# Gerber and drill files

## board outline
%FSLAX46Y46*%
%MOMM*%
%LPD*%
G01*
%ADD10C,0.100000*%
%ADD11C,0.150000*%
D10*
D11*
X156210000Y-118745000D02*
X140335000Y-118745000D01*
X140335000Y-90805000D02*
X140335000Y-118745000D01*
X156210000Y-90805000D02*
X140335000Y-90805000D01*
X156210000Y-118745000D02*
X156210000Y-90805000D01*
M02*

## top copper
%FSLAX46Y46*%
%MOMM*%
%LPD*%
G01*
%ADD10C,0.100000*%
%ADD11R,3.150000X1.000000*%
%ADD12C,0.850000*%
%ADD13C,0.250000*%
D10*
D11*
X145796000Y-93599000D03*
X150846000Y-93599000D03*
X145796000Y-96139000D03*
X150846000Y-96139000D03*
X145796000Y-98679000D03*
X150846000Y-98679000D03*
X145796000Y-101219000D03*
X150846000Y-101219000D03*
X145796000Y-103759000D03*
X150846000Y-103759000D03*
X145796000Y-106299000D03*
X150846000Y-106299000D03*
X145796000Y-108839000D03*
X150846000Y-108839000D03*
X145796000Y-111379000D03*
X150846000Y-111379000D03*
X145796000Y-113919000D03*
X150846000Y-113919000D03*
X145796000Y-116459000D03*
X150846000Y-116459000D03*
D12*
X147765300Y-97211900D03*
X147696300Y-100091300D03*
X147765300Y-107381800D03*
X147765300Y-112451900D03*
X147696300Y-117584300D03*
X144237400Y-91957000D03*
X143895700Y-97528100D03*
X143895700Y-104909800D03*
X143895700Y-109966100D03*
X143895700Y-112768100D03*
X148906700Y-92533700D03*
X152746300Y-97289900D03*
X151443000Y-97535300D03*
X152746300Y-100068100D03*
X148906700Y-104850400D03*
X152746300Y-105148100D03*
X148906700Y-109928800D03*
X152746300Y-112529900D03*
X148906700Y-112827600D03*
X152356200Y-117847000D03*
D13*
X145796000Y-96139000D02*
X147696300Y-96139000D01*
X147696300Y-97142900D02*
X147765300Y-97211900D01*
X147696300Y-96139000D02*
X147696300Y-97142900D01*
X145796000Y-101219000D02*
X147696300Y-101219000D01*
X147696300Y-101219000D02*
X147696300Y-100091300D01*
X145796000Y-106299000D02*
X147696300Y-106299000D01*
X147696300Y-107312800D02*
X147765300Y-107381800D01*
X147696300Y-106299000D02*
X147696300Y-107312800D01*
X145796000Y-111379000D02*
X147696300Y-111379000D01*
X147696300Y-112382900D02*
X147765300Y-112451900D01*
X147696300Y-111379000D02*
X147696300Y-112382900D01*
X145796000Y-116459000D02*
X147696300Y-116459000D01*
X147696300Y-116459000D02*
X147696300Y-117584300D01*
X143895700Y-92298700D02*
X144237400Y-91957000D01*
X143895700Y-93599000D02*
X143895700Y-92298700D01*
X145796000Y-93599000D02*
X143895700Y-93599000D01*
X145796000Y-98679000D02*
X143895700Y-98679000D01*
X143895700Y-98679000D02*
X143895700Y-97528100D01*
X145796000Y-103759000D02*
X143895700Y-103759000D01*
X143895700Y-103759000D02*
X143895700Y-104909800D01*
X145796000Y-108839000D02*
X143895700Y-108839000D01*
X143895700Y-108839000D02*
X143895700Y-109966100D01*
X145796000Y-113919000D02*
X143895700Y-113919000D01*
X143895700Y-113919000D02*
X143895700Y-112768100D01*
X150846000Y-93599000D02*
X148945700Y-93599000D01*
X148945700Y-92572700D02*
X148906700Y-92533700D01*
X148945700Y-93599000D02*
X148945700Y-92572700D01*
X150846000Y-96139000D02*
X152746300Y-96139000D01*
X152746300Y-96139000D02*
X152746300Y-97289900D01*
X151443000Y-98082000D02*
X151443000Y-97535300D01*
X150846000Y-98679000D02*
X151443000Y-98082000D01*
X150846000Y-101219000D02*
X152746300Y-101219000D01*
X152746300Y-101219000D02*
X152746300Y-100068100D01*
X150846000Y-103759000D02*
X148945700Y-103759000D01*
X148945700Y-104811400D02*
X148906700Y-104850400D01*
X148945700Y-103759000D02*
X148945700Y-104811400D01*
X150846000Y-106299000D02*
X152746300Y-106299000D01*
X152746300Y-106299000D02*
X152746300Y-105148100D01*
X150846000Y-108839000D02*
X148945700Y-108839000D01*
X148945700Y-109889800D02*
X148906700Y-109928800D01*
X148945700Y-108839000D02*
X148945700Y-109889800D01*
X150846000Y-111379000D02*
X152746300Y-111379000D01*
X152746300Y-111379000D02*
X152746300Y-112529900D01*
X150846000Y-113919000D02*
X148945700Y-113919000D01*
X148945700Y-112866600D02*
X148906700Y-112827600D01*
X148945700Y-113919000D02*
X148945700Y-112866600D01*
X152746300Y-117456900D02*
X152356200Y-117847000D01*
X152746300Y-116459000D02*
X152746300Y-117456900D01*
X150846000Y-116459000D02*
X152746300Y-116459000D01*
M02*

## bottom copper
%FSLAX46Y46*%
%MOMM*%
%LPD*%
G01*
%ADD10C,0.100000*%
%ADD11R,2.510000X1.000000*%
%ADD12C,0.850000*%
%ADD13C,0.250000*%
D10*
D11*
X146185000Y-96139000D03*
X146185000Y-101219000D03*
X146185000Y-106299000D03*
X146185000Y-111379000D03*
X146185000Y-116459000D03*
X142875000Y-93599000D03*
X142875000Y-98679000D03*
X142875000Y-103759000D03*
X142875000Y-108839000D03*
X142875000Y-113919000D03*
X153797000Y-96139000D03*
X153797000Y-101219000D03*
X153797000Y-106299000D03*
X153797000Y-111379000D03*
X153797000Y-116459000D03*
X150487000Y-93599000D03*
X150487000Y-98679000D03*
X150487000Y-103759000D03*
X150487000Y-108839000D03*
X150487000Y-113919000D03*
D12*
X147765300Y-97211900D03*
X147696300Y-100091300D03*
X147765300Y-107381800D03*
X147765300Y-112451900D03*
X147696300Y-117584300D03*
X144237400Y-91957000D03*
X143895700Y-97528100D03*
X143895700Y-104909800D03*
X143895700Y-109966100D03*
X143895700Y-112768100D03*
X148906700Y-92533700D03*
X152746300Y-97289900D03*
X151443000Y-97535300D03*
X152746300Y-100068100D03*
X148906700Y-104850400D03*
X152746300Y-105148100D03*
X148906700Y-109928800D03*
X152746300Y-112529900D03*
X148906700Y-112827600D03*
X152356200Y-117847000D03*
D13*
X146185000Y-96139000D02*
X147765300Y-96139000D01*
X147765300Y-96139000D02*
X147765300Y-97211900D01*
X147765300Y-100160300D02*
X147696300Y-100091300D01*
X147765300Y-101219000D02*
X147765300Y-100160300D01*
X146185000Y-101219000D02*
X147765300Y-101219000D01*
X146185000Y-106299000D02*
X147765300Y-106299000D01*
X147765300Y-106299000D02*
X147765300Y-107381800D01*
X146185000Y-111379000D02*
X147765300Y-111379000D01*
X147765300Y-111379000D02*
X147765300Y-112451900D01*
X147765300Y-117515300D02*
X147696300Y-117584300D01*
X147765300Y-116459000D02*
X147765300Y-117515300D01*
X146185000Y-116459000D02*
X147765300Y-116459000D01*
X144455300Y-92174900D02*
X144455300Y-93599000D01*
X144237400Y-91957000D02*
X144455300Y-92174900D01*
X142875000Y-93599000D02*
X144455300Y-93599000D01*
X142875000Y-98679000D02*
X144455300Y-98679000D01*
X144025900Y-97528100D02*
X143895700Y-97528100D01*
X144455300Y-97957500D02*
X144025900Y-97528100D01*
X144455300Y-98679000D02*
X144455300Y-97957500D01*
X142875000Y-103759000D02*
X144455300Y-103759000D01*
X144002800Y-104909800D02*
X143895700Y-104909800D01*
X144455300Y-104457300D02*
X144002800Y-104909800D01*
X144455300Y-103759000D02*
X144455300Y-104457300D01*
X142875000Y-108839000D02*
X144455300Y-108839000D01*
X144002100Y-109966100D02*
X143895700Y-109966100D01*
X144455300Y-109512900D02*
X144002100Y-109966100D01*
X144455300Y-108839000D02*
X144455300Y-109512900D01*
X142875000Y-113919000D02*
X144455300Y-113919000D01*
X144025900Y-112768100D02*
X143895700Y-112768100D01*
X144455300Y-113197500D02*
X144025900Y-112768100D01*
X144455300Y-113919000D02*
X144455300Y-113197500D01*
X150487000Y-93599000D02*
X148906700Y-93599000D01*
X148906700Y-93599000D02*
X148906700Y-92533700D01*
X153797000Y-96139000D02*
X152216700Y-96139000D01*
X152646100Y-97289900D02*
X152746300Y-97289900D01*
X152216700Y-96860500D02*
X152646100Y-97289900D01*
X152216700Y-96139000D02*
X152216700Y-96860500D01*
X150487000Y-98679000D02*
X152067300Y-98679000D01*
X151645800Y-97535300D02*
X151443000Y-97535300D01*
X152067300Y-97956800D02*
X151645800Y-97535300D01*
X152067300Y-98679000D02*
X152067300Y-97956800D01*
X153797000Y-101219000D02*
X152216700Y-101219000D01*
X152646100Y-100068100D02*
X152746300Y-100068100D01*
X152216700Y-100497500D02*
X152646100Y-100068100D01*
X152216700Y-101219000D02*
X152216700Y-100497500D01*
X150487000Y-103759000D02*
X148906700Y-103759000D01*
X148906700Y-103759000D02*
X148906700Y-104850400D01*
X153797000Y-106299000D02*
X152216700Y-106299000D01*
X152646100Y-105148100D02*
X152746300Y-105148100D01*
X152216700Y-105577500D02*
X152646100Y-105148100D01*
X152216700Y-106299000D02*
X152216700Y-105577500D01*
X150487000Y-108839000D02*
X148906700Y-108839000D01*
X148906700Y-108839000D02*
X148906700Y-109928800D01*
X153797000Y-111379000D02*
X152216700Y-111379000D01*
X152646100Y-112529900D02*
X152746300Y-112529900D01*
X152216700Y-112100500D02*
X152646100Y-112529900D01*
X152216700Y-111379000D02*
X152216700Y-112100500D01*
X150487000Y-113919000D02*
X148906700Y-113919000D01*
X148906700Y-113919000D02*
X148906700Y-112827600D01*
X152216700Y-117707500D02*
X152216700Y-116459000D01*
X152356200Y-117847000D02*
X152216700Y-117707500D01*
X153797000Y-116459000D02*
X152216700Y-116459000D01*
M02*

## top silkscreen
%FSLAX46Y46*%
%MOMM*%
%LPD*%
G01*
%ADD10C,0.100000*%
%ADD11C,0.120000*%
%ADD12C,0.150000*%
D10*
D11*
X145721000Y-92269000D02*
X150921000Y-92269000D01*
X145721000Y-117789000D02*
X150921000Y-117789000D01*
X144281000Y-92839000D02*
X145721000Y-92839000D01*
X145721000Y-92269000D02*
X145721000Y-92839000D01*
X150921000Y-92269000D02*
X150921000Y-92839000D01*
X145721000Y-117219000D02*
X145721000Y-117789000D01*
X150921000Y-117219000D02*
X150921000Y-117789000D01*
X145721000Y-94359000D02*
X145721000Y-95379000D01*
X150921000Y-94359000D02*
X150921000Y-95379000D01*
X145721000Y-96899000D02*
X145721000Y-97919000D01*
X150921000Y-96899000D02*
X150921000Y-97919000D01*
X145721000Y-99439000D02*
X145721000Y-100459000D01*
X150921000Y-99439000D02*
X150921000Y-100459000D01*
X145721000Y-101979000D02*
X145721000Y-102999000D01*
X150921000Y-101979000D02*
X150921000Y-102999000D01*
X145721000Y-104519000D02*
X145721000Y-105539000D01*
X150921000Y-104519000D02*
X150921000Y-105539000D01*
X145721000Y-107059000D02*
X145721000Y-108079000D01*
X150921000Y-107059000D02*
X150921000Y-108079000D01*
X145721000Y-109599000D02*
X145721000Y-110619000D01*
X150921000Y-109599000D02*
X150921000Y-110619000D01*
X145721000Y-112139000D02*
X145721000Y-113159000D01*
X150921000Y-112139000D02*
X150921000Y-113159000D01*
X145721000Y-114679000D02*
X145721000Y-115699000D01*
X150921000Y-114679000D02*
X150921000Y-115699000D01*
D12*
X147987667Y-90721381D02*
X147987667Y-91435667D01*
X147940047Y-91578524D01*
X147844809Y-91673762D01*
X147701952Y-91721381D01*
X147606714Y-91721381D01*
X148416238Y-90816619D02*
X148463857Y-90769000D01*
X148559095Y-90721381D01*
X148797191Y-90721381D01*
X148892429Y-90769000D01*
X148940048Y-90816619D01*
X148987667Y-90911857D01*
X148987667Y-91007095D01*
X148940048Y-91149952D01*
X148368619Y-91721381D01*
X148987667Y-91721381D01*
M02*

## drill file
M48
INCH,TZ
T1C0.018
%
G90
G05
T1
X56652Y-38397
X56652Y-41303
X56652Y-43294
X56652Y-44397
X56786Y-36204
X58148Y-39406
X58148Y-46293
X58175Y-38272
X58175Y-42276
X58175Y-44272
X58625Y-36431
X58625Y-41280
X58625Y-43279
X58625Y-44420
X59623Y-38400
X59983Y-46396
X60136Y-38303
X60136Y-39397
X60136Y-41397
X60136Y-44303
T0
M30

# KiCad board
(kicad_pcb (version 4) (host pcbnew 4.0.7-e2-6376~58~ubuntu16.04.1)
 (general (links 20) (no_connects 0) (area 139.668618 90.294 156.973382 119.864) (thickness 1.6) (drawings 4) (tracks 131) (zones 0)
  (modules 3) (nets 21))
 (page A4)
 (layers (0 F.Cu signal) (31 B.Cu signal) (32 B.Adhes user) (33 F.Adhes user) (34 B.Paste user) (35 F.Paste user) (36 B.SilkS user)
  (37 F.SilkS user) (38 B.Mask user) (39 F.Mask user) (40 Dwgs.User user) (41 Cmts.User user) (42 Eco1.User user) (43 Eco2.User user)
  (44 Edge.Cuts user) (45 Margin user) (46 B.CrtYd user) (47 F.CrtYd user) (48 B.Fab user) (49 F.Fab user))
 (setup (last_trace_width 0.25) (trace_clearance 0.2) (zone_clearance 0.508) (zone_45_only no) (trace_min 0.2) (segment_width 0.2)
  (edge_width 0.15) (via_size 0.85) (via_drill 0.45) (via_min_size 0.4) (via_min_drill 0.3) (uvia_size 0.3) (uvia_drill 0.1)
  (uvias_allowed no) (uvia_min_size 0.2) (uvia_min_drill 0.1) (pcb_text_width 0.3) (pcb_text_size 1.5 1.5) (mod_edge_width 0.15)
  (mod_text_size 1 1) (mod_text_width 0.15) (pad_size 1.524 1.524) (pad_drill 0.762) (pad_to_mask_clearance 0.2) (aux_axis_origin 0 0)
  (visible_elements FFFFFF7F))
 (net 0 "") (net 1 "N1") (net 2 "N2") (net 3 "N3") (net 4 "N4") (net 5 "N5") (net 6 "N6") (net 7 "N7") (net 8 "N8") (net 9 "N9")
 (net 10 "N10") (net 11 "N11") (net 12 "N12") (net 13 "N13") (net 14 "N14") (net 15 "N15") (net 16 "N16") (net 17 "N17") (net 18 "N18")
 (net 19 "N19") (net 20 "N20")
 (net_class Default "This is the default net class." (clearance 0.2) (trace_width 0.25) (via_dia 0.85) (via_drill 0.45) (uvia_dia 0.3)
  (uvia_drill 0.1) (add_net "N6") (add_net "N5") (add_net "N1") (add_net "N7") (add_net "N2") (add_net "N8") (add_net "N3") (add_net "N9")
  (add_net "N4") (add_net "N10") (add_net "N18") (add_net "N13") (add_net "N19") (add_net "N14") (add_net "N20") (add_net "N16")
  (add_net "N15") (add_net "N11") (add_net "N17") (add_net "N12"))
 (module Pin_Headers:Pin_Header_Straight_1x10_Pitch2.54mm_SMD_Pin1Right (layer B.Cu) (at 144.53 105.029 180)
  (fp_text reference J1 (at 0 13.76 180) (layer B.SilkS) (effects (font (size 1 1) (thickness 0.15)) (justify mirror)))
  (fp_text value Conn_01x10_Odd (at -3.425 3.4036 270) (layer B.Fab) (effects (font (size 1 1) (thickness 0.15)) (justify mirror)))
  (pad 2 smd rect (at -1.655 8.89 180) (size 2.51 1) (layers B.Cu B.Paste B.Mask) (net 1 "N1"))
  (pad 4 smd rect (at -1.655 3.81 180) (size 2.51 1) (layers B.Cu B.Paste B.Mask) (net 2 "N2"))
  (pad 6 smd rect (at -1.655 -1.27 180) (size 2.51 1) (layers B.Cu B.Paste B.Mask) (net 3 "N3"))
  (pad 8 smd rect (at -1.655 -6.35 180) (size 2.51 1) (layers B.Cu B.Paste B.Mask) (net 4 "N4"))
  (pad 10 smd rect (at -1.655 -11.43 180) (size 2.51 1) (layers B.Cu B.Paste B.Mask) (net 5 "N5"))
  (pad 1 smd rect (at 1.655 11.43 180) (size 2.51 1) (layers B.Cu B.Paste B.Mask) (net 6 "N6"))
  (pad 3 smd rect (at 1.655 6.35 180) (size 2.51 1) (layers B.Cu B.Paste B.Mask) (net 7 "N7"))
  (pad 5 smd rect (at 1.655 1.27 180) (size 2.51 1) (layers B.Cu B.Paste B.Mask) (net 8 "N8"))
  (pad 7 smd rect (at 1.655 -3.81 180) (size 2.51 1) (layers B.Cu B.Paste B.Mask) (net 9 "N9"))
  (pad 9 smd rect (at 1.655 -8.89 180) (size 2.51 1) (layers B.Cu B.Paste B.Mask) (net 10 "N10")))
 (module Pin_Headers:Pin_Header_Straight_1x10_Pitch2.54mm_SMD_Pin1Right (layer B.Cu) (at 152.142 105.029 180)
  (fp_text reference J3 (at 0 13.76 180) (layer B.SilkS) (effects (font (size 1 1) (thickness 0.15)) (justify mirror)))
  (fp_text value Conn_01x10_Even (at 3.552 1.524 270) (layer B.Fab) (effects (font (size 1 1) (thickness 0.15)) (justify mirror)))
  (pad 2 smd rect (at -1.655 8.89 180) (size 2.51 1) (layers B.Cu B.Paste B.Mask) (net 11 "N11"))
  (pad 4 smd rect (at -1.655 3.81 180) (size 2.51 1) (layers B.Cu B.Paste B.Mask) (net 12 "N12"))
  (pad 6 smd rect (at -1.655 -1.27 180) (size 2.51 1) (layers B.Cu B.Paste B.Mask) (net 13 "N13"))
  (pad 8 smd rect (at -1.655 -6.35 180) (size 2.51 1) (layers B.Cu B.Paste B.Mask) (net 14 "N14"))
  (pad 10 smd rect (at -1.655 -11.43 180) (size 2.51 1) (layers B.Cu B.Paste B.Mask) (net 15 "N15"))
  (pad 1 smd rect (at 1.655 11.43 180) (size 2.51 1) (layers B.Cu B.Paste B.Mask) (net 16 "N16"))
  (pad 3 smd rect (at 1.655 6.35 180) (size 2.51 1) (layers B.Cu B.Paste B.Mask) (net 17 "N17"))
  (pad 5 smd rect (at 1.655 1.27 180) (size 2.51 1) (layers B.Cu B.Paste B.Mask) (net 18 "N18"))
  (pad 7 smd rect (at 1.655 -3.81 180) (size 2.51 1) (layers B.Cu B.Paste B.Mask) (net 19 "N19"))
  (pad 9 smd rect (at 1.655 -8.89 180) (size 2.51 1) (layers B.Cu B.Paste B.Mask) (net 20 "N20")))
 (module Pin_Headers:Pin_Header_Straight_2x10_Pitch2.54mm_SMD (layer F.Cu) (at 148.321 105.029)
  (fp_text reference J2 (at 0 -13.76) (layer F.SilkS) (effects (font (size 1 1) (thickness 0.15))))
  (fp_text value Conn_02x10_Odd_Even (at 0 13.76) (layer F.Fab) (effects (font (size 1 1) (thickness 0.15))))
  (fp_line (start -2.6 -12.76) (end 2.6 -12.76) (layer F.SilkS) (width 0.12))
  (fp_line (start -2.6 12.76) (end 2.6 12.76) (layer F.SilkS) (width 0.12))
  (fp_line (start -4.04 -12.19) (end -2.6 -12.19) (layer F.SilkS) (width 0.12))
  (fp_line (start -2.6 -12.76) (end -2.6 -12.19) (layer F.SilkS) (width 0.12))
  (fp_line (start 2.6 -12.76) (end 2.6 -12.19) (layer F.SilkS) (width 0.12))
  (fp_line (start -2.6 12.19) (end -2.6 12.76) (layer F.SilkS) (width 0.12))
  (fp_line (start 2.6 12.19) (end 2.6 12.76) (layer F.SilkS) (width 0.12))
  (fp_line (start -2.6 -10.67) (end -2.6 -9.65) (layer F.SilkS) (width 0.12))
  (fp_line (start 2.6 -10.67) (end 2.6 -9.65) (layer F.SilkS) (width 0.12))
  (fp_line (start -2.6 -8.13) (end -2.6 -7.11) (layer F.SilkS) (width 0.12))
  (fp_line (start 2.6 -8.13) (end 2.6 -7.11) (layer F.SilkS) (width 0.12))
  (fp_line (start -2.6 -5.59) (end -2.6 -4.57) (layer F.SilkS) (width 0.12))
  (fp_line (start 2.6 -5.59) (end 2.6 -4.57) (layer F.SilkS) (width 0.12))
  (fp_line (start -2.6 -3.05) (end -2.6 -2.03) (layer F.SilkS) (width 0.12))
  (fp_line (start 2.6 -3.05) (end 2.6 -2.03) (layer F.SilkS) (width 0.12))
  (fp_line (start -2.6 -0.51) (end -2.6 0.51) (layer F.SilkS) (width 0.12))
  (fp_line (start 2.6 -0.51) (end 2.6 0.51) (layer F.SilkS) (width 0.12))
  (fp_line (start -2.6 2.03) (end -2.6 3.05) (layer F.SilkS) (width 0.12))
  (fp_line (start 2.6 2.03) (end 2.6 3.05) (layer F.SilkS) (width 0.12))
  (fp_line (start -2.6 4.57) (end -2.6 5.59) (layer F.SilkS) (width 0.12))
  (fp_line (start 2.6 4.57) (end 2.6 5.59) (layer F.SilkS) (width 0.12))
  (fp_line (start -2.6 7.11) (end -2.6 8.13) (layer F.SilkS) (width 0.12))
  (fp_line (start 2.6 7.11) (end 2.6 8.13) (layer F.SilkS) (width 0.12))
  (fp_line (start -2.6 9.65) (end -2.6 10.67) (layer F.SilkS) (width 0.12))
  (fp_line (start 2.6 9.65) (end 2.6 10.67) (layer F.SilkS) (width 0.12))
  (pad 1 smd rect (at -2.525 -11.43) (size 3.15 1) (layers F.Cu F.Paste F.Mask) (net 6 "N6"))
  (pad 2 smd rect (at 2.525 -11.43) (size 3.15 1) (layers F.Cu F.Paste F.Mask) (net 16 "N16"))
  (pad 3 smd rect (at -2.525 -8.89) (size 3.15 1) (layers F.Cu F.Paste F.Mask) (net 1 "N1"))
  (pad 4 smd rect (at 2.525 -8.89) (size 3.15 1) (layers F.Cu F.Paste F.Mask) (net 11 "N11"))
  (pad 5 smd rect (at -2.525 -6.35) (size 3.15 1) (layers F.Cu F.Paste F.Mask) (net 7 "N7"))
  (pad 6 smd rect (at 2.525 -6.35) (size 3.15 1) (layers F.Cu F.Paste F.Mask) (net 17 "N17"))
  (pad 7 smd rect (at -2.525 -3.81) (size 3.15 1) (layers F.Cu F.Paste F.Mask) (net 2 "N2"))
  (pad 8 smd rect (at 2.525 -3.81) (size 3.15 1) (layers F.Cu F.Paste F.Mask) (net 12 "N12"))
  (pad 9 smd rect (at -2.525 -1.27) (size 3.15 1) (layers F.Cu F.Paste F.Mask) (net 8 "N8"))
  (pad 10 smd rect (at 2.525 -1.27) (size 3.15 1) (layers F.Cu F.Paste F.Mask) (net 18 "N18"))
  (pad 11 smd rect (at -2.525 1.27) (size 3.15 1) (layers F.Cu F.Paste F.Mask) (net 3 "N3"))
  (pad 12 smd rect (at 2.525 1.27) (size 3.15 1) (layers F.Cu F.Paste F.Mask) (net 13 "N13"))
  (pad 13 smd rect (at -2.525 3.81) (size 3.15 1) (layers F.Cu F.Paste F.Mask) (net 9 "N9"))
  (pad 14 smd rect (at 2.525 3.81) (size 3.15 1) (layers F.Cu F.Paste F.Mask) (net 19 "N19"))
  (pad 15 smd rect (at -2.525 6.35) (size 3.15 1) (layers F.Cu F.Paste F.Mask) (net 4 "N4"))
  (pad 16 smd rect (at 2.525 6.35) (size 3.15 1) (layers F.Cu F.Paste F.Mask) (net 14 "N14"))
  (pad 17 smd rect (at -2.525 8.89) (size 3.15 1) (layers F.Cu F.Paste F.Mask) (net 10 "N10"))
  (pad 18 smd rect (at 2.525 8.89) (size 3.15 1) (layers F.Cu F.Paste F.Mask) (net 20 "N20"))
  (pad 19 smd rect (at -2.525 11.43) (size 3.15 1) (layers F.Cu F.Paste F.Mask) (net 5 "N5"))
  (pad 20 smd rect (at 2.525 11.43) (size 3.15 1) (layers F.Cu F.Paste F.Mask) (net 15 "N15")))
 (gr_line (start 156.21 118.745) (end 140.335 118.745) (layer Edge.Cuts) (width 0.15))
 (gr_line (start 140.335 90.805) (end 140.335 118.745) (layer Edge.Cuts) (width 0.15))
 (gr_line (start 156.21 90.805) (end 140.335 90.805) (layer Edge.Cuts) (width 0.15))
 (gr_line (start 156.21 118.745) (end 156.21 90.805) (layer Edge.Cuts) (width 0.15))
 (via (at 147.7653 97.2119) (size 0.85) (layers F.Cu B.Cu) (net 1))
 (segment (start 145.796 96.139) (end 147.6963 96.139) (width 0.25) (layer F.Cu) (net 1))
 (segment (start 146.185 96.139) (end 147.7653 96.139) (width 0.25) (layer B.Cu) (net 1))
 (segment (start 147.7653 96.139) (end 147.7653 97.2119) (width 0.25) (layer B.Cu) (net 1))
 (segment (start 147.6963 97.1429) (end 147.7653 97.2119) (width 0.25) (layer F.Cu) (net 1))
 (segment (start 147.6963 96.139) (end 147.6963 97.1429) (width 0.25) (layer F.Cu) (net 1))
 (via (at 147.6963 100.0913) (size 0.85) (layers F.Cu B.Cu) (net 2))
 (segment (start 145.796 101.219) (end 147.6963 101.219) (width 0.25) (layer F.Cu) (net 2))
 (segment (start 147.7653 100.1603) (end 147.6963 100.0913) (width 0.25) (layer B.Cu) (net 2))
 (segment (start 147.7653 101.219) (end 147.7653 100.1603) (width 0.25) (layer B.Cu) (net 2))
 (segment (start 147.6963 101.219) (end 147.6963 100.0913) (width 0.25) (layer F.Cu) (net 2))
 (segment (start 146.185 101.219) (end 147.7653 101.219) (width 0.25) (layer B.Cu) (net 2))
 (via (at 147.7653 107.3818) (size 0.85) (layers F.Cu B.Cu) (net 3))
 (segment (start 145.796 106.299) (end 147.6963 106.299) (width 0.25) (layer F.Cu) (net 3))
 (segment (start 146.185 106.299) (end 147.7653 106.299) (width 0.25) (layer B.Cu) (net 3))
 (segment (start 147.7653 106.299) (end 147.7653 107.3818) (width 0.25) (layer B.Cu) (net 3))
 (segment (start 147.6963 107.3128) (end 147.7653 107.3818) (width 0.25) (layer F.Cu) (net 3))
 (segment (start 147.6963 106.299) (end 147.6963 107.3128) (width 0.25) (layer F.Cu) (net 3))
 (via (at 147.7653 112.4519) (size 0.85) (layers F.Cu B.Cu) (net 4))
 (segment (start 145.796 111.379) (end 147.6963 111.379) (width 0.25) (layer F.Cu) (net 4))
 (segment (start 146.185 111.379) (end 147.7653 111.379) (width 0.25) (layer B.Cu) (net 4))
 (segment (start 147.7653 111.379) (end 147.7653 112.4519) (width 0.25) (layer B.Cu) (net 4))
 (segment (start 147.6963 112.3829) (end 147.7653 112.4519) (width 0.25) (layer F.Cu) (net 4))
 (segment (start 147.6963 111.379) (end 147.6963 112.3829) (width 0.25) (layer F.Cu) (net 4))
 (via (at 147.6963 117.5843) (size 0.85) (layers F.Cu B.Cu) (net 5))
 (segment (start 145.796 116.459) (end 147.6963 116.459) (width 0.25) (layer F.Cu) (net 5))
 (segment (start 147.7653 117.5153) (end 147.6963 117.5843) (width 0.25) (layer B.Cu) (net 5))
 (segment (start 147.7653 116.459) (end 147.7653 117.5153) (width 0.25) (layer B.Cu) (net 5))
 (segment (start 147.6963 116.459) (end 147.6963 117.5843) (width 0.25) (layer F.Cu) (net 5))
 (segment (start 146.185 116.459) (end 147.7653 116.459) (width 0.25) (layer B.Cu) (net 5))
 (via (at 144.2374 91.957) (size 0.85) (layers F.Cu B.Cu) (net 6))
 (segment (start 143.8957 92.2987) (end 144.2374 91.957) (width 0.25) (layer F.Cu) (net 6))
 (segment (start 143.8957 93.599) (end 143.8957 92.2987) (width 0.25) (layer F.Cu) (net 6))
 (segment (start 144.4553 92.1749) (end 144.4553 93.599) (width 0.25) (layer B.Cu) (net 6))
 (segment (start 144.2374 91.957) (end 144.4553 92.1749) (width 0.25) (layer B.Cu) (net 6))
 (segment (start 145.796 93.599) (end 143.8957 93.599) (width 0.25) (layer F.Cu) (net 6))
 (segment (start 142.875 93.599) (end 144.4553 93.599) (width 0.25) (layer B.Cu) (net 6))
 (via (at 143.8957 97.5281) (size 0.85) (layers F.Cu B.Cu) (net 7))
 (segment (start 145.796 98.679) (end 143.8957 98.679) (width 0.25) (layer F.Cu) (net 7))
 (segment (start 142.875 98.679) (end 144.4553 98.679) (width 0.25) (layer B.Cu) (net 7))
 (segment (start 144.0259 97.5281) (end 143.8957 97.5281) (width 0.25) (layer B.Cu) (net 7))
 (segment (start 144.4553 97.9575) (end 144.0259 97.5281) (width 0.25) (layer B.Cu) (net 7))
 (segment (start 144.4553 98.679) (end 144.4553 97.9575) (width 0.25) (layer B.Cu) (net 7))
 (segment (start 143.8957 98.679) (end 143.8957 97.5281) (width 0.25) (layer F.Cu) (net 7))
 (via (at 143.8957 104.9098) (size 0.85) (layers F.Cu B.Cu) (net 8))
 (segment (start 145.796 103.759) (end 143.8957 103.759) (width 0.25) (layer F.Cu) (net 8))
 (segment (start 142.875 103.759) (end 144.4553 103.759) (width 0.25) (layer B.Cu) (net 8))
 (segment (start 144.0028 104.9098) (end 143.8957 104.9098) (width 0.25) (layer B.Cu) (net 8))
 (segment (start 144.4553 104.4573) (end 144.0028 104.9098) (width 0.25) (layer B.Cu) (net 8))
 (segment (start 144.4553 103.759) (end 144.4553 104.4573) (width 0.25) (layer B.Cu) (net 8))
 (segment (start 143.8957 103.759) (end 143.8957 104.9098) (width 0.25) (layer F.Cu) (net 8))
 (via (at 143.8957 109.9661) (size 0.85) (layers F.Cu B.Cu) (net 9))
 (segment (start 145.796 108.839) (end 143.8957 108.839) (width 0.25) (layer F.Cu) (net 9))
 (segment (start 142.875 108.839) (end 144.4553 108.839) (width 0.25) (layer B.Cu) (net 9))
 (segment (start 144.0021 109.9661) (end 143.8957 109.9661) (width 0.25) (layer B.Cu) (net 9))
 (segment (start 144.4553 109.5129) (end 144.0021 109.9661) (width 0.25) (layer B.Cu) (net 9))
 (segment (start 144.4553 108.839) (end 144.4553 109.5129) (width 0.25) (layer B.Cu) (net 9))
 (segment (start 143.8957 108.839) (end 143.8957 109.9661) (width 0.25) (layer F.Cu) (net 9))
 (via (at 143.8957 112.7681) (size 0.85) (layers F.Cu B.Cu) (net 10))
 (segment (start 145.796 113.919) (end 143.8957 113.919) (width 0.25) (layer F.Cu) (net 10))
 (segment (start 142.875 113.919) (end 144.4553 113.919) (width 0.25) (layer B.Cu) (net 10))
 (segment (start 144.0259 112.7681) (end 143.8957 112.7681) (width 0.25) (layer B.Cu) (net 10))
 (segment (start 144.4553 113.1975) (end 144.0259 112.7681) (width 0.25) (layer B.Cu) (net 10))
 (segment (start 144.4553 113.919) (end 144.4553 113.1975) (width 0.25) (layer B.Cu) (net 10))
 (segment (start 143.8957 113.919) (end 143.8957 112.7681) (width 0.25) (layer F.Cu) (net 10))
 (via (at 148.9067 92.5337) (size 0.85) (layers F.Cu B.Cu) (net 16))
 (segment (start 150.846 93.599) (end 148.9457 93.599) (width 0.25) (layer F.Cu) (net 16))
 (segment (start 150.487 93.599) (end 148.9067 93.599) (width 0.25) (layer B.Cu) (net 16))
 (segment (start 148.9067 93.599) (end 148.9067 92.5337) (width 0.25) (layer B.Cu) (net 16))
 (segment (start 148.9457 92.5727) (end 148.9067 92.5337) (width 0.25) (layer F.Cu) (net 16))
 (segment (start 148.9457 93.599) (end 148.9457 92.5727) (width 0.25) (layer F.Cu) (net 16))
 (via (at 152.7463 97.2899) (size 0.85) (layers F.Cu B.Cu) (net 11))
 (segment (start 150.846 96.139) (end 152.7463 96.139) (width 0.25) (layer F.Cu) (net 11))
 (segment (start 153.797 96.139) (end 152.2167 96.139) (width 0.25) (layer B.Cu) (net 11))
 (segment (start 152.6461 97.2899) (end 152.7463 97.2899) (width 0.25) (layer B.Cu) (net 11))
 (segment (start 152.2167 96.8605) (end 152.6461 97.2899) (width 0.25) (layer B.Cu) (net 11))
 (segment (start 152.2167 96.139) (end 152.2167 96.8605) (width 0.25) (layer B.Cu) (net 11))
 (segment (start 152.7463 96.139) (end 152.7463 97.2899) (width 0.25) (layer F.Cu) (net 11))
 (via (at 151.443 97.5353) (size 0.85) (layers F.Cu B.Cu) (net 17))
 (segment (start 150.487 98.679) (end 152.0673 98.679) (width 0.25) (layer B.Cu) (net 17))
 (segment (start 151.6458 97.5353) (end 151.443 97.5353) (width 0.25) (layer B.Cu) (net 17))
 (segment (start 152.0673 97.9568) (end 151.6458 97.5353) (width 0.25) (layer B.Cu) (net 17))
 (segment (start 152.0673 98.679) (end 152.0673 97.9568) (width 0.25) (layer B.Cu) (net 17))
 (segment (start 151.443 98.082) (end 151.443 97.5353) (width 0.25) (layer F.Cu) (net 17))
 (segment (start 150.846 98.679) (end 151.443 98.082) (width 0.25) (layer F.Cu) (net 17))
 (via (at 152.7463 100.0681) (size 0.85) (layers F.Cu B.Cu) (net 12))
 (segment (start 150.846 101.219) (end 152.7463 101.219) (width 0.25) (layer F.Cu) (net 12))
 (segment (start 153.797 101.219) (end 152.2167 101.219) (width 0.25) (layer B.Cu) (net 12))
 (segment (start 152.6461 100.0681) (end 152.7463 100.0681) (width 0.25) (layer B.Cu) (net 12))
 (segment (start 152.2167 100.4975) (end 152.6461 100.0681) (width 0.25) (layer B.Cu) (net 12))
 (segment (start 152.2167 101.219) (end 152.2167 100.4975) (width 0.25) (layer B.Cu) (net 12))
 (segment (start 152.7463 101.219) (end 152.7463 100.0681) (width 0.25) (layer F.Cu) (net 12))
 (via (at 148.9067 104.8504) (size 0.85) (layers F.Cu B.Cu) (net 18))
 (segment (start 150.846 103.759) (end 148.9457 103.759) (width 0.25) (layer F.Cu) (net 18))
 (segment (start 150.487 103.759) (end 148.9067 103.759) (width 0.25) (layer B.Cu) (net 18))
 (segment (start 148.9067 103.759) (end 148.9067 104.8504) (width 0.25) (layer B.Cu) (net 18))
 (segment (start 148.9457 104.8114) (end 148.9067 104.8504) (width 0.25) (layer F.Cu) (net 18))
 (segment (start 148.9457 103.759) (end 148.9457 104.8114) (width 0.25) (layer F.Cu) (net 18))
 (via (at 152.7463 105.1481) (size 0.85) (layers F.Cu B.Cu) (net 13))
 (segment (start 150.846 106.299) (end 152.7463 106.299) (width 0.25) (layer F.Cu) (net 13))
 (segment (start 153.797 106.299) (end 152.2167 106.299) (width 0.25) (layer B.Cu) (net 13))
 (segment (start 152.6461 105.1481) (end 152.7463 105.1481) (width 0.25) (layer B.Cu) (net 13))
 (segment (start 152.2167 105.5775) (end 152.6461 105.1481) (width 0.25) (layer B.Cu) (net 13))
 (segment (start 152.2167 106.299) (end 152.2167 105.5775) (width 0.25) (layer B.Cu) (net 13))
 (segment (start 152.7463 106.299) (end 152.7463 105.1481) (width 0.25) (layer F.Cu) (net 13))
 (via (at 148.9067 109.9288) (size 0.85) (layers F.Cu B.Cu) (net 19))
 (segment (start 150.846 108.839) (end 148.9457 108.839) (width 0.25) (layer F.Cu) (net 19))
 (segment (start 150.487 108.839) (end 148.9067 108.839) (width 0.25) (layer B.Cu) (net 19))
 (segment (start 148.9067 108.839) (end 148.9067 109.9288) (width 0.25) (layer B.Cu) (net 19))
 (segment (start 148.9457 109.8898) (end 148.9067 109.9288) (width 0.25) (layer F.Cu) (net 19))
 (segment (start 148.9457 108.839) (end 148.9457 109.8898) (width 0.25) (layer F.Cu) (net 19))
 (via (at 152.7463 112.5299) (size 0.85) (layers F.Cu B.Cu) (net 14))
 (segment (start 150.846 111.379) (end 152.7463 111.379) (width 0.25) (layer F.Cu) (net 14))
 (segment (start 153.797 111.379) (end 152.2167 111.379) (width 0.25) (layer B.Cu) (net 14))
 (segment (start 152.6461 112.5299) (end 152.7463 112.5299) (width 0.25) (layer B.Cu) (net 14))
 (segment (start 152.2167 112.1005) (end 152.6461 112.5299) (width 0.25) (layer B.Cu) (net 14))
 (segment (start 152.2167 111.379) (end 152.2167 112.1005) (width 0.25) (layer B.Cu) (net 14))
 (segment (start 152.7463 111.379) (end 152.7463 112.5299) (width 0.25) (layer F.Cu) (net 14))
 (via (at 148.9067 112.8276) (size 0.85) (layers F.Cu B.Cu) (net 20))
 (segment (start 150.846 113.919) (end 148.9457 113.919) (width 0.25) (layer F.Cu) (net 20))
 (segment (start 150.487 113.919) (end 148.9067 113.919) (width 0.25) (layer B.Cu) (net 20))
 (segment (start 148.9067 113.919) (end 148.9067 112.8276) (width 0.25) (layer B.Cu) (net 20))
 (segment (start 148.9457 112.8666) (end 148.9067 112.8276) (width 0.25) (layer F.Cu) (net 20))
 (segment (start 148.9457 113.919) (end 148.9457 112.8666) (width 0.25) (layer F.Cu) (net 20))
 (via (at 152.3562 117.847) (size 0.85) (layers F.Cu B.Cu) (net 15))
 (segment (start 152.7463 117.4569) (end 152.3562 117.847) (width 0.25) (layer F.Cu) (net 15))
 (segment (start 152.7463 116.459) (end 152.7463 117.4569) (width 0.25) (layer F.Cu) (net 15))
 (segment (start 152.2167 117.7075) (end 152.2167 116.459) (width 0.25) (layer B.Cu) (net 15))
 (segment (start 152.3562 117.847) (end 152.2167 117.7075) (width 0.25) (layer B.Cu) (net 15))
 (segment (start 150.846 116.459) (end 152.7463 116.459) (width 0.25) (layer F.Cu) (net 15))
 (segment (start 153.797 116.459) (end 152.2167 116.459) (width 0.25) (layer B.Cu) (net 15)))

